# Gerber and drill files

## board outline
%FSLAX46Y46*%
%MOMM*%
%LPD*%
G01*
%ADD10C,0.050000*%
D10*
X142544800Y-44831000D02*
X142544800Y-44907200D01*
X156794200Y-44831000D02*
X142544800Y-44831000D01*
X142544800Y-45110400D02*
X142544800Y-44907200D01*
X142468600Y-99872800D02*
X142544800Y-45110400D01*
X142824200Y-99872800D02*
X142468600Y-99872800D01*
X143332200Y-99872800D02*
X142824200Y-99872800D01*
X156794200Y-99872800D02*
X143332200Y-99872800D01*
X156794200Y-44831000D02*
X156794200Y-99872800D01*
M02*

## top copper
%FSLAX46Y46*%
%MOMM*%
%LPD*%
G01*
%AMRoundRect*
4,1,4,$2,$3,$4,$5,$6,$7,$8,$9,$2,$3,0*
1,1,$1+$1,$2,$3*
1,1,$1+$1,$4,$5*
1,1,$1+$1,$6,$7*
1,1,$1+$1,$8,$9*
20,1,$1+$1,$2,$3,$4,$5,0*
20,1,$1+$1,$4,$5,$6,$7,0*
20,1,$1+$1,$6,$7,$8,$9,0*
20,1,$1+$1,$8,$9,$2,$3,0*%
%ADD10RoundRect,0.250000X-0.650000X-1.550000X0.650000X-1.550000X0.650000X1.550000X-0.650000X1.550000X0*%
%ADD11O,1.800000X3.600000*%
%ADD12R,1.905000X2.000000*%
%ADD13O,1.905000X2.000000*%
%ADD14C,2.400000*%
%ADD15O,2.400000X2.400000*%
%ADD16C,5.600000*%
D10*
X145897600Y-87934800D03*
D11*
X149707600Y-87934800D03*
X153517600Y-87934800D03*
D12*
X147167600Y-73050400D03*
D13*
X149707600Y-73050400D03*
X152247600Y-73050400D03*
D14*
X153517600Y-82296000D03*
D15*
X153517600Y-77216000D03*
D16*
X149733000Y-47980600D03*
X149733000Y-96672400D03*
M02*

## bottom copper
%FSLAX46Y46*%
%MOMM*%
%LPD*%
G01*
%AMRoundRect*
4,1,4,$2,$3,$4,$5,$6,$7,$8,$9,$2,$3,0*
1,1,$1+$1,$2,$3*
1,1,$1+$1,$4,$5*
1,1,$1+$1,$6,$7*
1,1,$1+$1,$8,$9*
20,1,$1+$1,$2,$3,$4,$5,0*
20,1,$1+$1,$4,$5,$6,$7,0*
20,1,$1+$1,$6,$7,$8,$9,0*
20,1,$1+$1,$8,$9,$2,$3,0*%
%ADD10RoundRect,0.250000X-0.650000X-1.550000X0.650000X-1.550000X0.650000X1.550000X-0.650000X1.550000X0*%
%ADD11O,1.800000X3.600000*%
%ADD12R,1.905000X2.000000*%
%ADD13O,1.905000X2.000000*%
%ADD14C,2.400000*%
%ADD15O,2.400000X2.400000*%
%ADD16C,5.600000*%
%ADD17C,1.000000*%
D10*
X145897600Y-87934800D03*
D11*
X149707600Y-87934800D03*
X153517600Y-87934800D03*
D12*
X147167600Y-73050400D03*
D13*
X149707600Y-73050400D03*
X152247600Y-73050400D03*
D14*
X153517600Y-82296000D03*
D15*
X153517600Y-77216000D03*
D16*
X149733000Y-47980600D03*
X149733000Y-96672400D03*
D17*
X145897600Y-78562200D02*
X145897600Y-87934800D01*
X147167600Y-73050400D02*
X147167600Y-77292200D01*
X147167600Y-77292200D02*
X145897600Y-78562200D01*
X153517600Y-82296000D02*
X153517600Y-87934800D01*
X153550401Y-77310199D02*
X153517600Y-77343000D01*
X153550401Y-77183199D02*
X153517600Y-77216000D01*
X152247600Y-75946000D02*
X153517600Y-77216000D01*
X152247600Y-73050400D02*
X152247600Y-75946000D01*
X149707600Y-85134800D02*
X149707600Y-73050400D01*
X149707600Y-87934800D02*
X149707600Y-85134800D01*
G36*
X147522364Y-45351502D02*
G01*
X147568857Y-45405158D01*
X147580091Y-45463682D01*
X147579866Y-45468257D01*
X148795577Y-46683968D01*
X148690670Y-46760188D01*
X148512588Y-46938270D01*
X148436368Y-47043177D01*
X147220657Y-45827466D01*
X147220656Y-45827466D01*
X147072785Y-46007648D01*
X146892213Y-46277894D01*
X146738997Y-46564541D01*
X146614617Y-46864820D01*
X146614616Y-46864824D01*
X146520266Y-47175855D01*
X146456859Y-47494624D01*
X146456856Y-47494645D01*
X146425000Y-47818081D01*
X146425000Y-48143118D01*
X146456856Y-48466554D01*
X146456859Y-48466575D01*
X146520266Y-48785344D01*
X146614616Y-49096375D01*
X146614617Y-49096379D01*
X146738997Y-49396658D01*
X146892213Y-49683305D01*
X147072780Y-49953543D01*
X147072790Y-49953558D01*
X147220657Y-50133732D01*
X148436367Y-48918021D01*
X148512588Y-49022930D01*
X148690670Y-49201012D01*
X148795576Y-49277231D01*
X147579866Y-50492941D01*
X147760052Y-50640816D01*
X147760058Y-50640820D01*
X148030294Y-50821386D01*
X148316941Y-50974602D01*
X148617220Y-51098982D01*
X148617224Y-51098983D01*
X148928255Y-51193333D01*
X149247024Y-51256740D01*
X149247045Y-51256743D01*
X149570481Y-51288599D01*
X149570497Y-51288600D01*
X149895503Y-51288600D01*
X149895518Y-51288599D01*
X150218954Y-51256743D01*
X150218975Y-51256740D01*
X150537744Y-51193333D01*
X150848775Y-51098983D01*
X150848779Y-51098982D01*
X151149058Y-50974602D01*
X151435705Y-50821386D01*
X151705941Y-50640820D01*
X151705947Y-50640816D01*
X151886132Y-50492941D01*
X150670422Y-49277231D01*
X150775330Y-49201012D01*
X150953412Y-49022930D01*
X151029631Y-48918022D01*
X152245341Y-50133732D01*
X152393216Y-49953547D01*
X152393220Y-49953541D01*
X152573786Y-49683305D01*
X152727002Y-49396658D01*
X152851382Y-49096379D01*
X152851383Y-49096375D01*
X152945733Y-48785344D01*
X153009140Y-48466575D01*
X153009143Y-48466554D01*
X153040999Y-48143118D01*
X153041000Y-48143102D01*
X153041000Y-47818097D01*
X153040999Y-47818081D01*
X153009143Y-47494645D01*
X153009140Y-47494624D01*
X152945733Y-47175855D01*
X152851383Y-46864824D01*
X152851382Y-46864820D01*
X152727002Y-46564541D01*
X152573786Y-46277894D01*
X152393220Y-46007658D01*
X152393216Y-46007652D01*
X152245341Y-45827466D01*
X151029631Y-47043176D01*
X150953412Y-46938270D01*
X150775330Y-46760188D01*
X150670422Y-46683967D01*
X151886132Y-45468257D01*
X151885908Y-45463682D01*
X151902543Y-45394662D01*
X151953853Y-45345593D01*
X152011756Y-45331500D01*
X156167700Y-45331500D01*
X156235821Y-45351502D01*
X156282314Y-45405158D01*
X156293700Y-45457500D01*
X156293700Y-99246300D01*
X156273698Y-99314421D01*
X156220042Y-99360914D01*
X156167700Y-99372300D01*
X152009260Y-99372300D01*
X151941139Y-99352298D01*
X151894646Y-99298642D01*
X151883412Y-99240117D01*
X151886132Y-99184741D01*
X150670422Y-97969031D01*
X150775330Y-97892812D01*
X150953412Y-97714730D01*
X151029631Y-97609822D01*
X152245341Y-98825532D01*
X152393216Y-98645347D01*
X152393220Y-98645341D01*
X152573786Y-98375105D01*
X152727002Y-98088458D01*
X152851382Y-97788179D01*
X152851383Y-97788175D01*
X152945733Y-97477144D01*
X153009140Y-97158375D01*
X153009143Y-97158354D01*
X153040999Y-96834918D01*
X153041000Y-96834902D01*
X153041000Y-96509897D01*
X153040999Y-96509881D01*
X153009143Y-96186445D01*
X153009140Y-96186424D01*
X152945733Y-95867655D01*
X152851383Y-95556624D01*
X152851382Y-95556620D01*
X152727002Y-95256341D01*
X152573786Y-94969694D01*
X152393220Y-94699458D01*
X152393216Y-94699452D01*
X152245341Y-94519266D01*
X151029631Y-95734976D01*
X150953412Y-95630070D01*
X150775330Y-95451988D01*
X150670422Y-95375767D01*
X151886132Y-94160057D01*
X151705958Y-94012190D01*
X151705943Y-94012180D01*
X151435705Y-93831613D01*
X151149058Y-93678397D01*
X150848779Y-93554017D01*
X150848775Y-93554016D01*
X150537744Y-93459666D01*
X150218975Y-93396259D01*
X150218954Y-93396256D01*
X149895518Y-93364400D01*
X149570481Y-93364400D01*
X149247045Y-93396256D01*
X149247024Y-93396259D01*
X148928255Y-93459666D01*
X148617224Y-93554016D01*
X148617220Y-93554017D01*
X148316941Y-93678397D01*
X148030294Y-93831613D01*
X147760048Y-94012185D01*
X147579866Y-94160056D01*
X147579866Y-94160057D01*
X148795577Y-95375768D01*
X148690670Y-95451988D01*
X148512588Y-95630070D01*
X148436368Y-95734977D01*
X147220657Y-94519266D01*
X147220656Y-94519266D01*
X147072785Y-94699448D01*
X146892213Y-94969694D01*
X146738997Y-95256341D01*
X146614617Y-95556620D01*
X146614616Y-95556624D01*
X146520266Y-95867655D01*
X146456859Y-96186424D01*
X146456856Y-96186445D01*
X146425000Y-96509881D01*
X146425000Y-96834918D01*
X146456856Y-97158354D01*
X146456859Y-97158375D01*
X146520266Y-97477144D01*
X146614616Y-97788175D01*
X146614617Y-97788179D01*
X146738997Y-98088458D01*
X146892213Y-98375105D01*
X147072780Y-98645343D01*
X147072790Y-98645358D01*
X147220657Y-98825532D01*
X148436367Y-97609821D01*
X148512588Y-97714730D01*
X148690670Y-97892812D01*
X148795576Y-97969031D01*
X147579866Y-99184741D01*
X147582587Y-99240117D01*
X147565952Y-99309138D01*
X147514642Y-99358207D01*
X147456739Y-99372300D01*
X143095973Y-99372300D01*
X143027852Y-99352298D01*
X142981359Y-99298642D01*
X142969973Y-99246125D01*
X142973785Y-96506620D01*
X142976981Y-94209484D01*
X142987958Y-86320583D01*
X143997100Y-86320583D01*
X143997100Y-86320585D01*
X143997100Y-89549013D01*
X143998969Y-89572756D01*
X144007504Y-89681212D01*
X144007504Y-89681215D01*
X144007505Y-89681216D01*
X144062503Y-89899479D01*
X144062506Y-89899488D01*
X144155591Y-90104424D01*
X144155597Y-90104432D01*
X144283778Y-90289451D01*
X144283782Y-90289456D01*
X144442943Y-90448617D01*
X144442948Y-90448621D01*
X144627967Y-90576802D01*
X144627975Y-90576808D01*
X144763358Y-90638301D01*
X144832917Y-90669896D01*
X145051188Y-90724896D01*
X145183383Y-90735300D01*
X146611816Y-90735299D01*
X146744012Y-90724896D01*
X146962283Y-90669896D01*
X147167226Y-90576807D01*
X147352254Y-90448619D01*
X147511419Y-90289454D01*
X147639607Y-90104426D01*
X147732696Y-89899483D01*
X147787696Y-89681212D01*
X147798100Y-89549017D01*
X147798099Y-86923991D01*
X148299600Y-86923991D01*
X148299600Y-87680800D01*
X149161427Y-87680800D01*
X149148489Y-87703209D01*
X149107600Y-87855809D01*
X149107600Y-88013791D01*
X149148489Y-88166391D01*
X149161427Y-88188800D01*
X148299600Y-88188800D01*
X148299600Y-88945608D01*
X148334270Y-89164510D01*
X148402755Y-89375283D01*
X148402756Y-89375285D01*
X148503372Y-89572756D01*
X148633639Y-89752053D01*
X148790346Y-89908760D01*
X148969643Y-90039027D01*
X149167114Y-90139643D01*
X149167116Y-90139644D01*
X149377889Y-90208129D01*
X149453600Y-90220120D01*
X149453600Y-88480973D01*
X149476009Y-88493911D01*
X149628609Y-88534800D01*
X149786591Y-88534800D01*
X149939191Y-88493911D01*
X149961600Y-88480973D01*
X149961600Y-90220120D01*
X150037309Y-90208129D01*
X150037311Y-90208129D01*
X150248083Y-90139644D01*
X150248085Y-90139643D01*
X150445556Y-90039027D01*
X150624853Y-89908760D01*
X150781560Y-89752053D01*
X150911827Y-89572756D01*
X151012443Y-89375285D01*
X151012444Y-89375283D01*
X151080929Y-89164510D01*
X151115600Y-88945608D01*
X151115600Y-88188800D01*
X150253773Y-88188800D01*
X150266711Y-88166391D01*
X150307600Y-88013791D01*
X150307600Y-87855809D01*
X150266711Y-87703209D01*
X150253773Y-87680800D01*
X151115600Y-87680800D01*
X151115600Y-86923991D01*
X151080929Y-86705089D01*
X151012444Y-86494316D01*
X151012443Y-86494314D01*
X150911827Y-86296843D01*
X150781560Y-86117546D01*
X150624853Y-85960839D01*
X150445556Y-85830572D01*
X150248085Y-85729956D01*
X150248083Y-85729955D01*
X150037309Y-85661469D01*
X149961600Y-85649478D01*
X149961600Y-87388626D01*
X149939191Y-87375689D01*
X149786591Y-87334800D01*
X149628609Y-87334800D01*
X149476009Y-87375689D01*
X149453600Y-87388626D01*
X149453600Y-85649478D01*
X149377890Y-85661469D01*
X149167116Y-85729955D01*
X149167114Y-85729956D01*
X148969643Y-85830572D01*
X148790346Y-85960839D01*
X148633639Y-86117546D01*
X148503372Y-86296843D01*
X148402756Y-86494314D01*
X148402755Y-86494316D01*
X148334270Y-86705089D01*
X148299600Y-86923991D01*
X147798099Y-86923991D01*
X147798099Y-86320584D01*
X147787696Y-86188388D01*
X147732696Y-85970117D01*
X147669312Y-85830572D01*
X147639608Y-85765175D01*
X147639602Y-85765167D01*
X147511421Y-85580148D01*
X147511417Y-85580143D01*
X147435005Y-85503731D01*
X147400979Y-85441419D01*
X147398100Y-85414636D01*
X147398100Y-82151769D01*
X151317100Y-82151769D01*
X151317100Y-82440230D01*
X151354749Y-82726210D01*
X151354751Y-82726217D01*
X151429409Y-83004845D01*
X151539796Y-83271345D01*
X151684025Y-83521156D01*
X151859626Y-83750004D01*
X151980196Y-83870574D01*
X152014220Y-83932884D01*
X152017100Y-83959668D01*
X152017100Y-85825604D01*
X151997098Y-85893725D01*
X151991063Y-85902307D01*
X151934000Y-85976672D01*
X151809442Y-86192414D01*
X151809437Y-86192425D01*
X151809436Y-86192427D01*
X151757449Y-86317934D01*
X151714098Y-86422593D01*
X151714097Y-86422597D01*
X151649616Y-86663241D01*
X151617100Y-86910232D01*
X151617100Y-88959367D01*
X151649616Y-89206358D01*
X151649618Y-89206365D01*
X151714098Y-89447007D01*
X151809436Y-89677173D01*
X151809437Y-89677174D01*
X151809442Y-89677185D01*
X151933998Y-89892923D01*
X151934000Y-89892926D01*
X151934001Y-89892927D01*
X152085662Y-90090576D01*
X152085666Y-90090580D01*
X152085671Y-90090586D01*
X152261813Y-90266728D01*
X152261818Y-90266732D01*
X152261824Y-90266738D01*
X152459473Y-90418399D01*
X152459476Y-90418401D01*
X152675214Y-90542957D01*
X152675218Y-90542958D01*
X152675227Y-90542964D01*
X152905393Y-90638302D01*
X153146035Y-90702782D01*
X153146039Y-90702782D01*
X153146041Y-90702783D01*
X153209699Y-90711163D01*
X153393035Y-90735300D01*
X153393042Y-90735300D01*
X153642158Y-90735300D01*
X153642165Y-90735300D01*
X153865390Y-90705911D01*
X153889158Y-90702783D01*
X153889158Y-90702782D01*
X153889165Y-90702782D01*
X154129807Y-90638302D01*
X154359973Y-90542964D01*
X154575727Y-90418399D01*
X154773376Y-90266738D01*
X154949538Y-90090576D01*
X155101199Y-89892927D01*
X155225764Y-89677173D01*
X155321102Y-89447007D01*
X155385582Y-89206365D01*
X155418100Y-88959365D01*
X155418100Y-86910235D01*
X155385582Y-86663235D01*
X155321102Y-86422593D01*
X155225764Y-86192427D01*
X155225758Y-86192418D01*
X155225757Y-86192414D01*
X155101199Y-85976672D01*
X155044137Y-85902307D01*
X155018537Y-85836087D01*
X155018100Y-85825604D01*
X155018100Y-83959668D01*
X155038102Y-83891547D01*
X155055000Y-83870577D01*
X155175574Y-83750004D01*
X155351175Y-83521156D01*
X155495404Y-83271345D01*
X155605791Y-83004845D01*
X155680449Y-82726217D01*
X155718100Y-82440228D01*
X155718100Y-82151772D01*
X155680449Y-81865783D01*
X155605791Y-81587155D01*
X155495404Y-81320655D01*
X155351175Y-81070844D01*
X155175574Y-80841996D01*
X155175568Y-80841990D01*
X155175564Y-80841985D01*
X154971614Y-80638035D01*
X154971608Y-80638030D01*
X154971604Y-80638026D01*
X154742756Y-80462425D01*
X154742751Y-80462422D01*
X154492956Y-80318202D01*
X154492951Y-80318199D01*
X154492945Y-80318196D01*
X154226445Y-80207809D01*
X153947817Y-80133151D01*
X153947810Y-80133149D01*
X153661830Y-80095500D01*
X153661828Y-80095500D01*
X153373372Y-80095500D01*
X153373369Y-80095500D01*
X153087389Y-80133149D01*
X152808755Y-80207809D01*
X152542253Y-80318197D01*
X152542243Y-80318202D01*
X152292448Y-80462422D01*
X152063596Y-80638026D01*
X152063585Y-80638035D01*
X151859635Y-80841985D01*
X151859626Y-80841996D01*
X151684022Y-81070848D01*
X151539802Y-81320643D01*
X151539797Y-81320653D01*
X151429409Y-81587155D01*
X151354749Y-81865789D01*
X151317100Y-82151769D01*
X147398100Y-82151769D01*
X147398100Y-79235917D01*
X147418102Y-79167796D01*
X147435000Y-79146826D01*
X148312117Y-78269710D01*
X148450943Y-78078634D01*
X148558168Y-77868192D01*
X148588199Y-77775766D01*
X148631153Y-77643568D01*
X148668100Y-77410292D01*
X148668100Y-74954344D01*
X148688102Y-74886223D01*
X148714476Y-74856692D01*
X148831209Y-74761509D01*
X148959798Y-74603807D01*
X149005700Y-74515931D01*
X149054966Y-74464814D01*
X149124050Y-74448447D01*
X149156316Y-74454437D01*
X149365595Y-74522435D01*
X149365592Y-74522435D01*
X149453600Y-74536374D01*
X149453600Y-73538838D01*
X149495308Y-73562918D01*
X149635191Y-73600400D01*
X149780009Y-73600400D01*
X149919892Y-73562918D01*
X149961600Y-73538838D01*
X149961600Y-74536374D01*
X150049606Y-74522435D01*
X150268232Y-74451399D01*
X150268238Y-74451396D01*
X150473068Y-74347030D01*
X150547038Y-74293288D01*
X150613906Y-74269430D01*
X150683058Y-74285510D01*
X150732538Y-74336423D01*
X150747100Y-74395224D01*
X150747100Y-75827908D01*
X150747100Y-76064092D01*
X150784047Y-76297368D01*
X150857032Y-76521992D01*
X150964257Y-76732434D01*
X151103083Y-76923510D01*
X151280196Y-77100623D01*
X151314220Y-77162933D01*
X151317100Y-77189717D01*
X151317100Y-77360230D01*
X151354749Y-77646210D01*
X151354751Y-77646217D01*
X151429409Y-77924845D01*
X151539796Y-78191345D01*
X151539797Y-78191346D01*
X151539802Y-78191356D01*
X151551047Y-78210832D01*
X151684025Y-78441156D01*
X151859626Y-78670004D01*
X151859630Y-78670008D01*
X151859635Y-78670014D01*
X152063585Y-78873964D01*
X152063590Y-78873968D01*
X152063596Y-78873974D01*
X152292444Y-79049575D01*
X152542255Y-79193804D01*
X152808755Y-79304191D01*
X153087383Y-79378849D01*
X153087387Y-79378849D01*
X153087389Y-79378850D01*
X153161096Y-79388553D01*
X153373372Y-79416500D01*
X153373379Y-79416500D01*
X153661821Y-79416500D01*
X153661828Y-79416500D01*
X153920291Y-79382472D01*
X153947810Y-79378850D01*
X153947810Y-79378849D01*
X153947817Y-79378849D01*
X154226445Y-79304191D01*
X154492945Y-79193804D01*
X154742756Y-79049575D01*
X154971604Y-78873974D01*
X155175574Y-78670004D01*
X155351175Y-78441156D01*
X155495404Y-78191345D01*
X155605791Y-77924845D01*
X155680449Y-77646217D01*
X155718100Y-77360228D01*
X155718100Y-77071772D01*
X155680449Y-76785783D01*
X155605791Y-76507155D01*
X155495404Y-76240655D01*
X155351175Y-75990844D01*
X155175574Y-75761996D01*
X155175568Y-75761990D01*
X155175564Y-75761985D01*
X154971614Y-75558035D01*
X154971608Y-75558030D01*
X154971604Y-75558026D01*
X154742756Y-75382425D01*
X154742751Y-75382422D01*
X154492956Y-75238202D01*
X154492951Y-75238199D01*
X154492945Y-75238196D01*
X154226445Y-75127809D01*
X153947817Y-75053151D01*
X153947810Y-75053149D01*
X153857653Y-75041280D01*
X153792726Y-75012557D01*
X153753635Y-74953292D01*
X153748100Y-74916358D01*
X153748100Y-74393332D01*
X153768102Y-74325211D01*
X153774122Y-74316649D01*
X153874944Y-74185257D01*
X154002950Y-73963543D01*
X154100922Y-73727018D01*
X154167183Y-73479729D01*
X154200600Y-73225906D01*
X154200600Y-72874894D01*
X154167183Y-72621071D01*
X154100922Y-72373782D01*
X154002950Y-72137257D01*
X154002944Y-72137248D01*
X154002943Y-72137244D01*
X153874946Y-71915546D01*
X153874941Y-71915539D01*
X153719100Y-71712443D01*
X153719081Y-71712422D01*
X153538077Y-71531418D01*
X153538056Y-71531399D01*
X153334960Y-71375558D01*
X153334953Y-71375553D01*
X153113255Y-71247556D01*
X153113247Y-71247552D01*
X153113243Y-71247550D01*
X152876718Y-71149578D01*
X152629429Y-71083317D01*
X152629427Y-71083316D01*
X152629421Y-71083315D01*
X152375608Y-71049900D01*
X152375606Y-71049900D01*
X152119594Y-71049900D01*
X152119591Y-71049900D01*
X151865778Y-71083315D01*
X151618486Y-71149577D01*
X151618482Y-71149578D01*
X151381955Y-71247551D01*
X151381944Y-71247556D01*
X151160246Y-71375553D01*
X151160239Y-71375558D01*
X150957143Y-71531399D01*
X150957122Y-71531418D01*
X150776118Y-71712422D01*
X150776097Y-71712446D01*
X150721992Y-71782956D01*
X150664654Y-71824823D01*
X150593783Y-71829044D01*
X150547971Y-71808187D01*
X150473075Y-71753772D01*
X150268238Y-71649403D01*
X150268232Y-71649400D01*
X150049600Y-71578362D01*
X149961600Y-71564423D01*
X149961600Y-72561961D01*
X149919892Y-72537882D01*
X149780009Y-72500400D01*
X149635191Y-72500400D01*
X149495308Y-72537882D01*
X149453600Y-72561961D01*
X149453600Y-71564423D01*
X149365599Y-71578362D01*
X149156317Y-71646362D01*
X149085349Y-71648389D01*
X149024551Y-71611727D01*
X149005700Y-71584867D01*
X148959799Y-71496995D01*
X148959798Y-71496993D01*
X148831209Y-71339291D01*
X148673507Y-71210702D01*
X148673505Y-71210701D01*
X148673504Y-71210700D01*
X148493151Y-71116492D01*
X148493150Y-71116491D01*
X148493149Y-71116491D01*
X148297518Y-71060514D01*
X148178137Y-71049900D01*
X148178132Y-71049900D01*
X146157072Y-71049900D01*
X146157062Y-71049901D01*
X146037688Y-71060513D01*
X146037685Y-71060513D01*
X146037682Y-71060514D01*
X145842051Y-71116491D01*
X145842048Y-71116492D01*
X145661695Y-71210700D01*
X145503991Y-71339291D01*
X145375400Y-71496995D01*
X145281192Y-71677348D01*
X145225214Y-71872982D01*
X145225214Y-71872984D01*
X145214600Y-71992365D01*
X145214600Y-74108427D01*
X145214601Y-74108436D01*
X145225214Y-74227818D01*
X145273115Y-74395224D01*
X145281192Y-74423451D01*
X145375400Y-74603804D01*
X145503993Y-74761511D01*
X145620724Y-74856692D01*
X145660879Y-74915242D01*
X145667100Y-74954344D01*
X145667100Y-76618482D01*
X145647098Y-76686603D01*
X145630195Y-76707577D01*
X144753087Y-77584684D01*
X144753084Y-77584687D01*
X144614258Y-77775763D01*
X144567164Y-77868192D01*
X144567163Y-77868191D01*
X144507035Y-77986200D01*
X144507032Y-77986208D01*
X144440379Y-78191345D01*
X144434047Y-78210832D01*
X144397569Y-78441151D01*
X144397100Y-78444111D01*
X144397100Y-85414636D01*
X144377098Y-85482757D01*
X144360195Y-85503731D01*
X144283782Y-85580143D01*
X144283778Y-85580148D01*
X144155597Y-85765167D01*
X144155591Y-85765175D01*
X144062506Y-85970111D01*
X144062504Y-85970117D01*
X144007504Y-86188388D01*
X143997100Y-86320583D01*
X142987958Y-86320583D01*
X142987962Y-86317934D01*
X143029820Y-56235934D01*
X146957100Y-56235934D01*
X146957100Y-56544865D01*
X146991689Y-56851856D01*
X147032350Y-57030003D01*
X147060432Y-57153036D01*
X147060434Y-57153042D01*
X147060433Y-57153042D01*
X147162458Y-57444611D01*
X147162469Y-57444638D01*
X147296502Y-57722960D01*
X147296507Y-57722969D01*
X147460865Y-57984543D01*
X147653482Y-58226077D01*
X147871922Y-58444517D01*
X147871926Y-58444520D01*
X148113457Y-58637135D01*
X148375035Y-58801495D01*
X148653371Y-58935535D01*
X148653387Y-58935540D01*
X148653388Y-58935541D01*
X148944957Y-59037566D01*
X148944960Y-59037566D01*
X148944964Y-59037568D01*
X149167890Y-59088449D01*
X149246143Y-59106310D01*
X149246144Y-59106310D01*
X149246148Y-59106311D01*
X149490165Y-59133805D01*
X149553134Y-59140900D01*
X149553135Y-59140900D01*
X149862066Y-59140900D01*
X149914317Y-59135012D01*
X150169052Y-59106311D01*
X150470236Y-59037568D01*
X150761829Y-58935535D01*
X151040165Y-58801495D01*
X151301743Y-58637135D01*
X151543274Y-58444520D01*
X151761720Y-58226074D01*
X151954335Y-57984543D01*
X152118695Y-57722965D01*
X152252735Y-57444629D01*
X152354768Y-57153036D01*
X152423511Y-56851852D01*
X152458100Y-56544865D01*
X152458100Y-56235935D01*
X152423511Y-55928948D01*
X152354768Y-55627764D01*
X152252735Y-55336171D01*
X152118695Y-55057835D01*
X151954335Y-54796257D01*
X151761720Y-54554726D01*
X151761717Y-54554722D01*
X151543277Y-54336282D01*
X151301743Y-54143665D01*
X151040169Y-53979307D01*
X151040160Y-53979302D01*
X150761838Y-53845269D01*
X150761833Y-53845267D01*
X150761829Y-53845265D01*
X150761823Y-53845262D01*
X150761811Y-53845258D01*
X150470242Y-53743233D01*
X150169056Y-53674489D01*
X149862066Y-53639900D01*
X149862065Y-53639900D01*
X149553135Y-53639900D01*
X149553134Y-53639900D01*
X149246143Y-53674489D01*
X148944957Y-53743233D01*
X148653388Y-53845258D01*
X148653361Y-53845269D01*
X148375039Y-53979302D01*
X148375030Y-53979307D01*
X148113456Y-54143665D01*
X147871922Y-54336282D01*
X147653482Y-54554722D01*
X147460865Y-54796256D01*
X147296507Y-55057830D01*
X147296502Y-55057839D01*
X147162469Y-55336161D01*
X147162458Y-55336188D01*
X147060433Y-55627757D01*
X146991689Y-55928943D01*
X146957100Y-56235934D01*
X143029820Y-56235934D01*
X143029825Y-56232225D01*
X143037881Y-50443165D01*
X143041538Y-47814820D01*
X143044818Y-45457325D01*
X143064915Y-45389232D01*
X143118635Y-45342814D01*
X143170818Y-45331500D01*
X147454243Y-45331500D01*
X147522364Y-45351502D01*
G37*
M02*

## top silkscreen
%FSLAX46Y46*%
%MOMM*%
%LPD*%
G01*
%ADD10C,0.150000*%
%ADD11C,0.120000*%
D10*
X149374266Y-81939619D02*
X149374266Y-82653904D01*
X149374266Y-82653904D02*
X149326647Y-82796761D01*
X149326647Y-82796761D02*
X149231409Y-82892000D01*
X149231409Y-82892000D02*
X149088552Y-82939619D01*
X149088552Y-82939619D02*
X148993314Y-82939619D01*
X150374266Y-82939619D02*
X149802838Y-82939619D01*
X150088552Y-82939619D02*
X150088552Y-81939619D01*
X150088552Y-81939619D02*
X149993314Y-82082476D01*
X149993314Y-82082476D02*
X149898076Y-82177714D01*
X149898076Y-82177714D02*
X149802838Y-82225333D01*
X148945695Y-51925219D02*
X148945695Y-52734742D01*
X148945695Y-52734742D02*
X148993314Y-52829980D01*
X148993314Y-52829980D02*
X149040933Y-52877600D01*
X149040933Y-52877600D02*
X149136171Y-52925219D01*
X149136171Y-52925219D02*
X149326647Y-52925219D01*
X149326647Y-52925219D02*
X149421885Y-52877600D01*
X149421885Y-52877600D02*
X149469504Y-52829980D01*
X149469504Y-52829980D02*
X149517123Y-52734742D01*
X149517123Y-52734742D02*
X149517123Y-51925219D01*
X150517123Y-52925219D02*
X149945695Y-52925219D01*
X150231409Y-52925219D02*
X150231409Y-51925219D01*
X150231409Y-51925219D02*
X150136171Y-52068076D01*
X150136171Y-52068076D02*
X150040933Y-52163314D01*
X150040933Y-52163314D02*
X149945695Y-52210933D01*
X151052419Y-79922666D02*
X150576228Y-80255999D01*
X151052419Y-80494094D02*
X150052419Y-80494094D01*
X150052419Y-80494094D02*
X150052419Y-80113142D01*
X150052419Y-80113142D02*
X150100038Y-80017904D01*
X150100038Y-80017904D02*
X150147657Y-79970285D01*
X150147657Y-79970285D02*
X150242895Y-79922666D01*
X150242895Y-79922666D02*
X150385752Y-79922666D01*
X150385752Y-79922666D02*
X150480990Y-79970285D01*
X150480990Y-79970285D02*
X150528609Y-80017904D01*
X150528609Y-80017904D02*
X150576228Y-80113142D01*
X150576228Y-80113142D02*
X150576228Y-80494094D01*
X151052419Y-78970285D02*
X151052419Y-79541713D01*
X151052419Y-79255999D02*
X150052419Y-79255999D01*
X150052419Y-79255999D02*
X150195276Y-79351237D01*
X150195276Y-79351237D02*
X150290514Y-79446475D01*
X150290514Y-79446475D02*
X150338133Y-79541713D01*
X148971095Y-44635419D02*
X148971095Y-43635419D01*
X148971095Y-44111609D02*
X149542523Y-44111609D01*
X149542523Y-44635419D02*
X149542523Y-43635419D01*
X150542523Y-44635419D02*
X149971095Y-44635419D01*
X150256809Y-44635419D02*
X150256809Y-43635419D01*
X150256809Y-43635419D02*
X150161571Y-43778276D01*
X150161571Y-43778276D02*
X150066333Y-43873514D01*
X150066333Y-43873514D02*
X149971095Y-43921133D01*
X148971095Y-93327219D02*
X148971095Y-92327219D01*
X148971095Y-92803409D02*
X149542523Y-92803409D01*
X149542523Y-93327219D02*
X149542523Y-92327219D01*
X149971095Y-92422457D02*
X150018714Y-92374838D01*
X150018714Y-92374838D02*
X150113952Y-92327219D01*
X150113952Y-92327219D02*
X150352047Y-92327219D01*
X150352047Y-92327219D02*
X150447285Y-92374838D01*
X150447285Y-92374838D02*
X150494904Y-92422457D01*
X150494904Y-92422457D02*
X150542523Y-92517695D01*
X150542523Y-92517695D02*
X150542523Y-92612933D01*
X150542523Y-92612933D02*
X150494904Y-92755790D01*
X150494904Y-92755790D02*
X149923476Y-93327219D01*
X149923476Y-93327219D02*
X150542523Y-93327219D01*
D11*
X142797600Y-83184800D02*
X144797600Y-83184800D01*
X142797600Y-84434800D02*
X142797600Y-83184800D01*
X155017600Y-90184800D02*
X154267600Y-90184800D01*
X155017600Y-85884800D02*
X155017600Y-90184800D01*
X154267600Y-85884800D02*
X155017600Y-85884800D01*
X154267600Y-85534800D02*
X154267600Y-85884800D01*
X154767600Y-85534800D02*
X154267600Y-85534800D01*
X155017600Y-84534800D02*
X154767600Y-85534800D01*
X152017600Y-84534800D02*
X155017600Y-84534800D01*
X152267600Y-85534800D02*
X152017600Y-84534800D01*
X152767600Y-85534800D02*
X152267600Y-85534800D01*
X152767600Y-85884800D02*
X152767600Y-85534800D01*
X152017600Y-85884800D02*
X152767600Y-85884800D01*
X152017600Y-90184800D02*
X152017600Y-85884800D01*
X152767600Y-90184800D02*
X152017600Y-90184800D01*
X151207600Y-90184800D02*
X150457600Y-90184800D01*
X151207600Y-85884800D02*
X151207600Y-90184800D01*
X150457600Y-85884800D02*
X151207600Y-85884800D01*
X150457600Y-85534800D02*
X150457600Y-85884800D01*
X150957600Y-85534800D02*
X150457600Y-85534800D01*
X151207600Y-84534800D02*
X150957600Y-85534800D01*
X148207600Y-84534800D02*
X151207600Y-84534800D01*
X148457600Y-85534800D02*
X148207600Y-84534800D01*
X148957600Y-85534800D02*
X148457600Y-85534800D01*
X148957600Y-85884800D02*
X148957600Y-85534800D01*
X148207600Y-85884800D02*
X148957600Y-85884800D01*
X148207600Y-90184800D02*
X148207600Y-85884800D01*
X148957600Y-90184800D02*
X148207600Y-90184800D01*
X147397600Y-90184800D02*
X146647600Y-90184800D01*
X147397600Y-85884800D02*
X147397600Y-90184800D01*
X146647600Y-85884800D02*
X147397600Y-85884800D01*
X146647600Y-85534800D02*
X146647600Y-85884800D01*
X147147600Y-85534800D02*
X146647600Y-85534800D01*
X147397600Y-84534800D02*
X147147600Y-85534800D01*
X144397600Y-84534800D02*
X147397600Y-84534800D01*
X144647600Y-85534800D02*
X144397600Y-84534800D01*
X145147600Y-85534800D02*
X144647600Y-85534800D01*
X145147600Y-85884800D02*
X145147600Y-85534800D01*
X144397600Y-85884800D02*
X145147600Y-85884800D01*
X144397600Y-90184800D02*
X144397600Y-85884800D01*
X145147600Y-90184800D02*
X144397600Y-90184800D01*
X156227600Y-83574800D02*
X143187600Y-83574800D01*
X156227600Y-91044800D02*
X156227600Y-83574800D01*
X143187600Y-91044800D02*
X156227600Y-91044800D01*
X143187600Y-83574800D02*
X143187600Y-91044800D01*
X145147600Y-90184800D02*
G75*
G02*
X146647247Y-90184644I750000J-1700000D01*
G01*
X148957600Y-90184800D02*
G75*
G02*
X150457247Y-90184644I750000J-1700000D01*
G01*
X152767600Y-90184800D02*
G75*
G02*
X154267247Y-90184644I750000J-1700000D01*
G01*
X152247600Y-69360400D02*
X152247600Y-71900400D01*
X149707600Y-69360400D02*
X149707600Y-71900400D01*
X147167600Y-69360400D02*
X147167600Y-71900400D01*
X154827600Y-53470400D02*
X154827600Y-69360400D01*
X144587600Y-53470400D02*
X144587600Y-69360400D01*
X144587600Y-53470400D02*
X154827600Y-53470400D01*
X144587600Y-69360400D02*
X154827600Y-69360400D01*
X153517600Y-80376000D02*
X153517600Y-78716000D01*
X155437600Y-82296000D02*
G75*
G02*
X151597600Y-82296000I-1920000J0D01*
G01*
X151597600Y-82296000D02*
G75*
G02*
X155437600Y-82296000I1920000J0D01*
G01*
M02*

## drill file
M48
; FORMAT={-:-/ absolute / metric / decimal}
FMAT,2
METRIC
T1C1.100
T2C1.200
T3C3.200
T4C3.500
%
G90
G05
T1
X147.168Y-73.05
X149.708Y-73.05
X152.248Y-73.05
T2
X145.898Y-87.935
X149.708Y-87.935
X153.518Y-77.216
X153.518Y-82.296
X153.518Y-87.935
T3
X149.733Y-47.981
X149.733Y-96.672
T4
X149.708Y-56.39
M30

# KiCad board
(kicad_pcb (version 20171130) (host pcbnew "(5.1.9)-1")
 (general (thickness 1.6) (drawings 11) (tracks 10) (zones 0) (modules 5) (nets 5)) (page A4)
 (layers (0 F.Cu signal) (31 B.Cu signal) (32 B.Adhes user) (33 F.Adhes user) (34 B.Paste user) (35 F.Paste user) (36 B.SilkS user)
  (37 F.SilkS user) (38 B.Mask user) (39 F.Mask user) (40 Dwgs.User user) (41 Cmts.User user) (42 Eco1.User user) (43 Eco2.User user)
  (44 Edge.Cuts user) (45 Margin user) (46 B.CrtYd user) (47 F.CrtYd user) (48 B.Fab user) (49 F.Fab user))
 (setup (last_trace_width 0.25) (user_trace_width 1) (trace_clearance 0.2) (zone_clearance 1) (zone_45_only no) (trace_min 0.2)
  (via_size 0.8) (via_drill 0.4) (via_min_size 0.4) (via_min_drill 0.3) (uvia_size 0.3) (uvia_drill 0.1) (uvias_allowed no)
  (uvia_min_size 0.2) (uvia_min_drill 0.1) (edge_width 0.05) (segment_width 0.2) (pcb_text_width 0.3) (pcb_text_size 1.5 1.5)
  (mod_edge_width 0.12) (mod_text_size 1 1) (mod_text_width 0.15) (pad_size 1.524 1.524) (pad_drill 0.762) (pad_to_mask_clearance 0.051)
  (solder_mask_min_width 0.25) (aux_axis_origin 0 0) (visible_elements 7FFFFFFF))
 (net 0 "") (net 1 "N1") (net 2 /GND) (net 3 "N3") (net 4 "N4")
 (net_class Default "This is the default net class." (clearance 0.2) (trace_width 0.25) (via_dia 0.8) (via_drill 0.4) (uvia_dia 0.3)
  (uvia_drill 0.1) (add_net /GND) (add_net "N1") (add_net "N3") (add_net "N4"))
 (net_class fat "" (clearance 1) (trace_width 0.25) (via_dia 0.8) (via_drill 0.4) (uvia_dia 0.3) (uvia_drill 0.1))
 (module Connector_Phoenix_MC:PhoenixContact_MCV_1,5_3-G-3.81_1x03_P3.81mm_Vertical (layer F.Cu) (at 145.8976 87.9348)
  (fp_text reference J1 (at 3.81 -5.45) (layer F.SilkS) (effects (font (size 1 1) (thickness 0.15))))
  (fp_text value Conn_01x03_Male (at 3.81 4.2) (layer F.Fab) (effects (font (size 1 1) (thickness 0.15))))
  (fp_line (start -3.1 -4.75) (end -1.1 -4.75) (layer F.SilkS) (width 0.12))
  (fp_line (start -3.1 -3.5) (end -3.1 -4.75) (layer F.SilkS) (width 0.12))
  (fp_line (start 9.12 2.25) (end 8.37 2.25) (layer F.SilkS) (width 0.12))
  (fp_line (start 9.12 -2.05) (end 9.12 2.25) (layer F.SilkS) (width 0.12))
  (fp_line (start 8.37 -2.05) (end 9.12 -2.05) (layer F.SilkS) (width 0.12))
  (fp_line (start 8.37 -2.4) (end 8.37 -2.05) (layer F.SilkS) (width 0.12))
  (fp_line (start 8.87 -2.4) (end 8.37 -2.4) (layer F.SilkS) (width 0.12))
  (fp_line (start 9.12 -3.4) (end 8.87 -2.4) (layer F.SilkS) (width 0.12))
  (fp_line (start 6.12 -3.4) (end 9.12 -3.4) (layer F.SilkS) (width 0.12))
  (fp_line (start 6.37 -2.4) (end 6.12 -3.4) (layer F.SilkS) (width 0.12))
  (fp_line (start 6.87 -2.4) (end 6.37 -2.4) (layer F.SilkS) (width 0.12))
  (fp_line (start 6.87 -2.05) (end 6.87 -2.4) (layer F.SilkS) (width 0.12))
  (fp_line (start 6.12 -2.05) (end 6.87 -2.05) (layer F.SilkS) (width 0.12))
  (fp_line (start 6.12 2.25) (end 6.12 -2.05) (layer F.SilkS) (width 0.12))
  (fp_line (start 6.87 2.25) (end 6.12 2.25) (layer F.SilkS) (width 0.12))
  (fp_line (start 5.31 2.25) (end 4.56 2.25) (layer F.SilkS) (width 0.12))
  (fp_line (start 5.31 -2.05) (end 5.31 2.25) (layer F.SilkS) (width 0.12))
  (fp_line (start 4.56 -2.05) (end 5.31 -2.05) (layer F.SilkS) (width 0.12))
  (fp_line (start 4.56 -2.4) (end 4.56 -2.05) (layer F.SilkS) (width 0.12))
  (fp_line (start 5.06 -2.4) (end 4.56 -2.4) (layer F.SilkS) (width 0.12))
  (fp_line (start 5.31 -3.4) (end 5.06 -2.4) (layer F.SilkS) (width 0.12))
  (fp_line (start 2.31 -3.4) (end 5.31 -3.4) (layer F.SilkS) (width 0.12))
  (fp_line (start 2.56 -2.4) (end 2.31 -3.4) (layer F.SilkS) (width 0.12))
  (fp_line (start 3.06 -2.4) (end 2.56 -2.4) (layer F.SilkS) (width 0.12))
  (fp_line (start 3.06 -2.05) (end 3.06 -2.4) (layer F.SilkS) (width 0.12))
  (fp_line (start 2.31 -2.05) (end 3.06 -2.05) (layer F.SilkS) (width 0.12))
  (fp_line (start 2.31 2.25) (end 2.31 -2.05) (layer F.SilkS) (width 0.12))
  (fp_line (start 3.06 2.25) (end 2.31 2.25) (layer F.SilkS) (width 0.12))
  (fp_line (start 1.5 2.25) (end 0.75 2.25) (layer F.SilkS) (width 0.12))
  (fp_line (start 1.5 -2.05) (end 1.5 2.25) (layer F.SilkS) (width 0.12))
  (fp_line (start 0.75 -2.05) (end 1.5 -2.05) (layer F.SilkS) (width 0.12))
  (fp_line (start 0.75 -2.4) (end 0.75 -2.05) (layer F.SilkS) (width 0.12))
  (fp_line (start 1.25 -2.4) (end 0.75 -2.4) (layer F.SilkS) (width 0.12))
  (fp_line (start 1.5 -3.4) (end 1.25 -2.4) (layer F.SilkS) (width 0.12))
  (fp_line (start -1.5 -3.4) (end 1.5 -3.4) (layer F.SilkS) (width 0.12))
  (fp_line (start -1.25 -2.4) (end -1.5 -3.4) (layer F.SilkS) (width 0.12))
  (fp_line (start -0.75 -2.4) (end -1.25 -2.4) (layer F.SilkS) (width 0.12))
  (fp_line (start -0.75 -2.05) (end -0.75 -2.4) (layer F.SilkS) (width 0.12))
  (fp_line (start -1.5 -2.05) (end -0.75 -2.05) (layer F.SilkS) (width 0.12))
  (fp_line (start -1.5 2.25) (end -1.5 -2.05) (layer F.SilkS) (width 0.12))
  (fp_line (start -0.75 2.25) (end -1.5 2.25) (layer F.SilkS) (width 0.12))
  (fp_line (start 10.33 -4.36) (end -2.71 -4.36) (layer F.SilkS) (width 0.12))
  (fp_line (start 10.33 3.11) (end 10.33 -4.36) (layer F.SilkS) (width 0.12))
  (fp_line (start -2.71 3.11) (end 10.33 3.11) (layer F.SilkS) (width 0.12))
  (fp_line (start -2.71 -4.36) (end -2.71 3.11) (layer F.SilkS) (width 0.12))
  (fp_arc (start 0 3.95) (end -0.75 2.25) (angle 47.6) (layer F.SilkS) (width 0.12))
  (fp_arc (start 3.81 3.95) (end 3.06 2.25) (angle 47.6) (layer F.SilkS) (width 0.12))
  (fp_arc (start 7.62 3.95) (end 6.87 2.25) (angle 47.6) (layer F.SilkS) (width 0.12))
  (pad 1 thru_hole roundrect (at 0 0) (size 1.8 3.6) (drill 1.2) (layers *.Cu *.Mask) (roundrect_rratio 0.1388888888888889) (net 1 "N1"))
  (pad 2 thru_hole oval (at 3.81 0) (size 1.8 3.6) (drill 1.2) (layers *.Cu *.Mask) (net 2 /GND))
  (pad 3 thru_hole oval (at 7.62 0) (size 1.8 3.6) (drill 1.2) (layers *.Cu *.Mask) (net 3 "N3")))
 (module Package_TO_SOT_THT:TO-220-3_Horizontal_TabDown (layer F.Cu) (at 147.1676 73.0504)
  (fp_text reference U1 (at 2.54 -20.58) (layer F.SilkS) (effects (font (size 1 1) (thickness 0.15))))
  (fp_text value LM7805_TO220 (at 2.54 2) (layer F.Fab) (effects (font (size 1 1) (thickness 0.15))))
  (fp_line (start 5.08 -3.69) (end 5.08 -1.15) (layer F.SilkS) (width 0.12))
  (fp_line (start 2.54 -3.69) (end 2.54 -1.15) (layer F.SilkS) (width 0.12))
  (fp_line (start 0 -3.69) (end 0 -1.15) (layer F.SilkS) (width 0.12))
  (fp_line (start 7.66 -19.58) (end 7.66 -3.69) (layer F.SilkS) (width 0.12))
  (fp_line (start -2.58 -19.58) (end -2.58 -3.69) (layer F.SilkS) (width 0.12))
  (fp_line (start -2.58 -19.58) (end 7.66 -19.58) (layer F.SilkS) (width 0.12))
  (fp_line (start -2.58 -3.69) (end 7.66 -3.69) (layer F.SilkS) (width 0.12))
  (pad "" np_thru_hole oval (at 2.54 -16.66) (size 3.5 3.5) (drill 3.5) (layers *.Cu *.Mask))
  (pad 1 thru_hole rect (at 0 0) (size 1.905 2) (drill 1.1) (layers *.Cu *.Mask) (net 1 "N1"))
  (pad 2 thru_hole oval (at 2.54 0) (size 1.905 2) (drill 1.1) (layers *.Cu *.Mask) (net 2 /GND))
  (pad 3 thru_hole oval (at 5.08 0) (size 1.905 2) (drill 1.1) (layers *.Cu *.Mask) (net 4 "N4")))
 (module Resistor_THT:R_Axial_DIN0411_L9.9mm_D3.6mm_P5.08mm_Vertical (layer F.Cu) (at 153.5176 82.296 90)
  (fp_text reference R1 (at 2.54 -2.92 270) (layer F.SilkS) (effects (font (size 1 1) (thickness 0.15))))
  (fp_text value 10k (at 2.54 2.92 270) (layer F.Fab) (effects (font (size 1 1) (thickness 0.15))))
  (fp_line (start 1.92 0) (end 3.58 0) (layer F.SilkS) (width 0.12))
  (fp_circle (center 0 0) (end 1.92 0) (layer F.SilkS) (width 0.12))
  (pad 1 thru_hole circle (at 0 0 90) (size 2.4 2.4) (drill 1.2) (layers *.Cu *.Mask) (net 3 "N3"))
  (pad 2 thru_hole oval (at 5.08 0 90) (size 2.4 2.4) (drill 1.2) (layers *.Cu *.Mask) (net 4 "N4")))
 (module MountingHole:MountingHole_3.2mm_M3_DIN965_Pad (layer F.Cu) (at 149.733 47.9806)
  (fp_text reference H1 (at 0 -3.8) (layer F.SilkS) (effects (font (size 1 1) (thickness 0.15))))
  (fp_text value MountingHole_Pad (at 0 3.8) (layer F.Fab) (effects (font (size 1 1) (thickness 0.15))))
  (pad 1 thru_hole circle (at 0 0) (size 5.6 5.6) (drill 3.2) (layers *.Cu *.Mask) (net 2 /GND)))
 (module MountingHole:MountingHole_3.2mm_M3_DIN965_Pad (layer F.Cu) (at 149.733 96.6724)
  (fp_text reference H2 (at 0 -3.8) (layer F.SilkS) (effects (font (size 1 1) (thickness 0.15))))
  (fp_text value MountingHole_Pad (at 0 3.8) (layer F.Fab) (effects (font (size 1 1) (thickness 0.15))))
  (pad 1 thru_hole circle (at 0 0) (size 5.6 5.6) (drill 3.2) (layers *.Cu *.Mask) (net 2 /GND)))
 (gr_line (start 142.5448 44.831) (end 142.5448 44.9072) (layer Edge.Cuts) (width 0.05))
 (gr_line (start 156.7942 44.831) (end 142.5448 44.831) (layer Edge.Cuts) (width 0.05))
 (gr_line (start 142.5448 45.1104) (end 142.5448 44.9072) (layer Edge.Cuts) (width 0.05))
 (gr_line (start 142.4686 99.8728) (end 142.5448 45.1104) (layer Edge.Cuts) (width 0.05))
 (gr_line (start 142.8242 99.8728) (end 142.4686 99.8728) (layer Edge.Cuts) (width 0.05))
 (gr_line (start 143.3322 99.8728) (end 142.8242 99.8728) (layer Edge.Cuts) (width 0.05))
 (gr_line (start 156.7942 99.8728) (end 143.3322 99.8728) (layer Edge.Cuts) (width 0.05))
 (gr_line (start 156.7942 44.831) (end 156.7942 99.8728) (layer Edge.Cuts) (width 0.05))
 (segment (start 145.8976 78.5622) (end 145.8976 87.9348) (width 1) (layer B.Cu) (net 1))
 (segment (start 147.1676 73.0504) (end 147.1676 77.2922) (width 1) (layer B.Cu) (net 1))
 (segment (start 147.1676 77.2922) (end 145.8976 78.5622) (width 1) (layer B.Cu) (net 1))
 (segment (start 153.5176 82.296) (end 153.5176 87.9348) (width 1) (layer B.Cu) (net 3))
 (segment (start 153.550401 77.310199) (end 153.5176 77.343) (width 1) (layer B.Cu) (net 4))
 (segment (start 153.550401 77.183199) (end 153.5176 77.216) (width 1) (layer B.Cu) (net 4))
 (segment (start 152.2476 75.946) (end 153.5176 77.216) (width 1) (layer B.Cu) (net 4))
 (segment (start 152.2476 73.0504) (end 152.2476 75.946) (width 1) (layer B.Cu) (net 4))
 (segment (start 149.7076 85.1348) (end 149.7076 73.0504) (width 1) (layer B.Cu) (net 2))
 (segment (start 149.7076 87.9348) (end 149.7076 85.1348) (width 1) (layer B.Cu) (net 2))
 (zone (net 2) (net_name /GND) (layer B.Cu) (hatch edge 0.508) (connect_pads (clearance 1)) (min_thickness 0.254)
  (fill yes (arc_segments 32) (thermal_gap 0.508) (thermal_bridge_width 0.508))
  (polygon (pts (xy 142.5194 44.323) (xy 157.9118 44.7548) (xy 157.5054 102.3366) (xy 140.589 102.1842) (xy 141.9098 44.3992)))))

